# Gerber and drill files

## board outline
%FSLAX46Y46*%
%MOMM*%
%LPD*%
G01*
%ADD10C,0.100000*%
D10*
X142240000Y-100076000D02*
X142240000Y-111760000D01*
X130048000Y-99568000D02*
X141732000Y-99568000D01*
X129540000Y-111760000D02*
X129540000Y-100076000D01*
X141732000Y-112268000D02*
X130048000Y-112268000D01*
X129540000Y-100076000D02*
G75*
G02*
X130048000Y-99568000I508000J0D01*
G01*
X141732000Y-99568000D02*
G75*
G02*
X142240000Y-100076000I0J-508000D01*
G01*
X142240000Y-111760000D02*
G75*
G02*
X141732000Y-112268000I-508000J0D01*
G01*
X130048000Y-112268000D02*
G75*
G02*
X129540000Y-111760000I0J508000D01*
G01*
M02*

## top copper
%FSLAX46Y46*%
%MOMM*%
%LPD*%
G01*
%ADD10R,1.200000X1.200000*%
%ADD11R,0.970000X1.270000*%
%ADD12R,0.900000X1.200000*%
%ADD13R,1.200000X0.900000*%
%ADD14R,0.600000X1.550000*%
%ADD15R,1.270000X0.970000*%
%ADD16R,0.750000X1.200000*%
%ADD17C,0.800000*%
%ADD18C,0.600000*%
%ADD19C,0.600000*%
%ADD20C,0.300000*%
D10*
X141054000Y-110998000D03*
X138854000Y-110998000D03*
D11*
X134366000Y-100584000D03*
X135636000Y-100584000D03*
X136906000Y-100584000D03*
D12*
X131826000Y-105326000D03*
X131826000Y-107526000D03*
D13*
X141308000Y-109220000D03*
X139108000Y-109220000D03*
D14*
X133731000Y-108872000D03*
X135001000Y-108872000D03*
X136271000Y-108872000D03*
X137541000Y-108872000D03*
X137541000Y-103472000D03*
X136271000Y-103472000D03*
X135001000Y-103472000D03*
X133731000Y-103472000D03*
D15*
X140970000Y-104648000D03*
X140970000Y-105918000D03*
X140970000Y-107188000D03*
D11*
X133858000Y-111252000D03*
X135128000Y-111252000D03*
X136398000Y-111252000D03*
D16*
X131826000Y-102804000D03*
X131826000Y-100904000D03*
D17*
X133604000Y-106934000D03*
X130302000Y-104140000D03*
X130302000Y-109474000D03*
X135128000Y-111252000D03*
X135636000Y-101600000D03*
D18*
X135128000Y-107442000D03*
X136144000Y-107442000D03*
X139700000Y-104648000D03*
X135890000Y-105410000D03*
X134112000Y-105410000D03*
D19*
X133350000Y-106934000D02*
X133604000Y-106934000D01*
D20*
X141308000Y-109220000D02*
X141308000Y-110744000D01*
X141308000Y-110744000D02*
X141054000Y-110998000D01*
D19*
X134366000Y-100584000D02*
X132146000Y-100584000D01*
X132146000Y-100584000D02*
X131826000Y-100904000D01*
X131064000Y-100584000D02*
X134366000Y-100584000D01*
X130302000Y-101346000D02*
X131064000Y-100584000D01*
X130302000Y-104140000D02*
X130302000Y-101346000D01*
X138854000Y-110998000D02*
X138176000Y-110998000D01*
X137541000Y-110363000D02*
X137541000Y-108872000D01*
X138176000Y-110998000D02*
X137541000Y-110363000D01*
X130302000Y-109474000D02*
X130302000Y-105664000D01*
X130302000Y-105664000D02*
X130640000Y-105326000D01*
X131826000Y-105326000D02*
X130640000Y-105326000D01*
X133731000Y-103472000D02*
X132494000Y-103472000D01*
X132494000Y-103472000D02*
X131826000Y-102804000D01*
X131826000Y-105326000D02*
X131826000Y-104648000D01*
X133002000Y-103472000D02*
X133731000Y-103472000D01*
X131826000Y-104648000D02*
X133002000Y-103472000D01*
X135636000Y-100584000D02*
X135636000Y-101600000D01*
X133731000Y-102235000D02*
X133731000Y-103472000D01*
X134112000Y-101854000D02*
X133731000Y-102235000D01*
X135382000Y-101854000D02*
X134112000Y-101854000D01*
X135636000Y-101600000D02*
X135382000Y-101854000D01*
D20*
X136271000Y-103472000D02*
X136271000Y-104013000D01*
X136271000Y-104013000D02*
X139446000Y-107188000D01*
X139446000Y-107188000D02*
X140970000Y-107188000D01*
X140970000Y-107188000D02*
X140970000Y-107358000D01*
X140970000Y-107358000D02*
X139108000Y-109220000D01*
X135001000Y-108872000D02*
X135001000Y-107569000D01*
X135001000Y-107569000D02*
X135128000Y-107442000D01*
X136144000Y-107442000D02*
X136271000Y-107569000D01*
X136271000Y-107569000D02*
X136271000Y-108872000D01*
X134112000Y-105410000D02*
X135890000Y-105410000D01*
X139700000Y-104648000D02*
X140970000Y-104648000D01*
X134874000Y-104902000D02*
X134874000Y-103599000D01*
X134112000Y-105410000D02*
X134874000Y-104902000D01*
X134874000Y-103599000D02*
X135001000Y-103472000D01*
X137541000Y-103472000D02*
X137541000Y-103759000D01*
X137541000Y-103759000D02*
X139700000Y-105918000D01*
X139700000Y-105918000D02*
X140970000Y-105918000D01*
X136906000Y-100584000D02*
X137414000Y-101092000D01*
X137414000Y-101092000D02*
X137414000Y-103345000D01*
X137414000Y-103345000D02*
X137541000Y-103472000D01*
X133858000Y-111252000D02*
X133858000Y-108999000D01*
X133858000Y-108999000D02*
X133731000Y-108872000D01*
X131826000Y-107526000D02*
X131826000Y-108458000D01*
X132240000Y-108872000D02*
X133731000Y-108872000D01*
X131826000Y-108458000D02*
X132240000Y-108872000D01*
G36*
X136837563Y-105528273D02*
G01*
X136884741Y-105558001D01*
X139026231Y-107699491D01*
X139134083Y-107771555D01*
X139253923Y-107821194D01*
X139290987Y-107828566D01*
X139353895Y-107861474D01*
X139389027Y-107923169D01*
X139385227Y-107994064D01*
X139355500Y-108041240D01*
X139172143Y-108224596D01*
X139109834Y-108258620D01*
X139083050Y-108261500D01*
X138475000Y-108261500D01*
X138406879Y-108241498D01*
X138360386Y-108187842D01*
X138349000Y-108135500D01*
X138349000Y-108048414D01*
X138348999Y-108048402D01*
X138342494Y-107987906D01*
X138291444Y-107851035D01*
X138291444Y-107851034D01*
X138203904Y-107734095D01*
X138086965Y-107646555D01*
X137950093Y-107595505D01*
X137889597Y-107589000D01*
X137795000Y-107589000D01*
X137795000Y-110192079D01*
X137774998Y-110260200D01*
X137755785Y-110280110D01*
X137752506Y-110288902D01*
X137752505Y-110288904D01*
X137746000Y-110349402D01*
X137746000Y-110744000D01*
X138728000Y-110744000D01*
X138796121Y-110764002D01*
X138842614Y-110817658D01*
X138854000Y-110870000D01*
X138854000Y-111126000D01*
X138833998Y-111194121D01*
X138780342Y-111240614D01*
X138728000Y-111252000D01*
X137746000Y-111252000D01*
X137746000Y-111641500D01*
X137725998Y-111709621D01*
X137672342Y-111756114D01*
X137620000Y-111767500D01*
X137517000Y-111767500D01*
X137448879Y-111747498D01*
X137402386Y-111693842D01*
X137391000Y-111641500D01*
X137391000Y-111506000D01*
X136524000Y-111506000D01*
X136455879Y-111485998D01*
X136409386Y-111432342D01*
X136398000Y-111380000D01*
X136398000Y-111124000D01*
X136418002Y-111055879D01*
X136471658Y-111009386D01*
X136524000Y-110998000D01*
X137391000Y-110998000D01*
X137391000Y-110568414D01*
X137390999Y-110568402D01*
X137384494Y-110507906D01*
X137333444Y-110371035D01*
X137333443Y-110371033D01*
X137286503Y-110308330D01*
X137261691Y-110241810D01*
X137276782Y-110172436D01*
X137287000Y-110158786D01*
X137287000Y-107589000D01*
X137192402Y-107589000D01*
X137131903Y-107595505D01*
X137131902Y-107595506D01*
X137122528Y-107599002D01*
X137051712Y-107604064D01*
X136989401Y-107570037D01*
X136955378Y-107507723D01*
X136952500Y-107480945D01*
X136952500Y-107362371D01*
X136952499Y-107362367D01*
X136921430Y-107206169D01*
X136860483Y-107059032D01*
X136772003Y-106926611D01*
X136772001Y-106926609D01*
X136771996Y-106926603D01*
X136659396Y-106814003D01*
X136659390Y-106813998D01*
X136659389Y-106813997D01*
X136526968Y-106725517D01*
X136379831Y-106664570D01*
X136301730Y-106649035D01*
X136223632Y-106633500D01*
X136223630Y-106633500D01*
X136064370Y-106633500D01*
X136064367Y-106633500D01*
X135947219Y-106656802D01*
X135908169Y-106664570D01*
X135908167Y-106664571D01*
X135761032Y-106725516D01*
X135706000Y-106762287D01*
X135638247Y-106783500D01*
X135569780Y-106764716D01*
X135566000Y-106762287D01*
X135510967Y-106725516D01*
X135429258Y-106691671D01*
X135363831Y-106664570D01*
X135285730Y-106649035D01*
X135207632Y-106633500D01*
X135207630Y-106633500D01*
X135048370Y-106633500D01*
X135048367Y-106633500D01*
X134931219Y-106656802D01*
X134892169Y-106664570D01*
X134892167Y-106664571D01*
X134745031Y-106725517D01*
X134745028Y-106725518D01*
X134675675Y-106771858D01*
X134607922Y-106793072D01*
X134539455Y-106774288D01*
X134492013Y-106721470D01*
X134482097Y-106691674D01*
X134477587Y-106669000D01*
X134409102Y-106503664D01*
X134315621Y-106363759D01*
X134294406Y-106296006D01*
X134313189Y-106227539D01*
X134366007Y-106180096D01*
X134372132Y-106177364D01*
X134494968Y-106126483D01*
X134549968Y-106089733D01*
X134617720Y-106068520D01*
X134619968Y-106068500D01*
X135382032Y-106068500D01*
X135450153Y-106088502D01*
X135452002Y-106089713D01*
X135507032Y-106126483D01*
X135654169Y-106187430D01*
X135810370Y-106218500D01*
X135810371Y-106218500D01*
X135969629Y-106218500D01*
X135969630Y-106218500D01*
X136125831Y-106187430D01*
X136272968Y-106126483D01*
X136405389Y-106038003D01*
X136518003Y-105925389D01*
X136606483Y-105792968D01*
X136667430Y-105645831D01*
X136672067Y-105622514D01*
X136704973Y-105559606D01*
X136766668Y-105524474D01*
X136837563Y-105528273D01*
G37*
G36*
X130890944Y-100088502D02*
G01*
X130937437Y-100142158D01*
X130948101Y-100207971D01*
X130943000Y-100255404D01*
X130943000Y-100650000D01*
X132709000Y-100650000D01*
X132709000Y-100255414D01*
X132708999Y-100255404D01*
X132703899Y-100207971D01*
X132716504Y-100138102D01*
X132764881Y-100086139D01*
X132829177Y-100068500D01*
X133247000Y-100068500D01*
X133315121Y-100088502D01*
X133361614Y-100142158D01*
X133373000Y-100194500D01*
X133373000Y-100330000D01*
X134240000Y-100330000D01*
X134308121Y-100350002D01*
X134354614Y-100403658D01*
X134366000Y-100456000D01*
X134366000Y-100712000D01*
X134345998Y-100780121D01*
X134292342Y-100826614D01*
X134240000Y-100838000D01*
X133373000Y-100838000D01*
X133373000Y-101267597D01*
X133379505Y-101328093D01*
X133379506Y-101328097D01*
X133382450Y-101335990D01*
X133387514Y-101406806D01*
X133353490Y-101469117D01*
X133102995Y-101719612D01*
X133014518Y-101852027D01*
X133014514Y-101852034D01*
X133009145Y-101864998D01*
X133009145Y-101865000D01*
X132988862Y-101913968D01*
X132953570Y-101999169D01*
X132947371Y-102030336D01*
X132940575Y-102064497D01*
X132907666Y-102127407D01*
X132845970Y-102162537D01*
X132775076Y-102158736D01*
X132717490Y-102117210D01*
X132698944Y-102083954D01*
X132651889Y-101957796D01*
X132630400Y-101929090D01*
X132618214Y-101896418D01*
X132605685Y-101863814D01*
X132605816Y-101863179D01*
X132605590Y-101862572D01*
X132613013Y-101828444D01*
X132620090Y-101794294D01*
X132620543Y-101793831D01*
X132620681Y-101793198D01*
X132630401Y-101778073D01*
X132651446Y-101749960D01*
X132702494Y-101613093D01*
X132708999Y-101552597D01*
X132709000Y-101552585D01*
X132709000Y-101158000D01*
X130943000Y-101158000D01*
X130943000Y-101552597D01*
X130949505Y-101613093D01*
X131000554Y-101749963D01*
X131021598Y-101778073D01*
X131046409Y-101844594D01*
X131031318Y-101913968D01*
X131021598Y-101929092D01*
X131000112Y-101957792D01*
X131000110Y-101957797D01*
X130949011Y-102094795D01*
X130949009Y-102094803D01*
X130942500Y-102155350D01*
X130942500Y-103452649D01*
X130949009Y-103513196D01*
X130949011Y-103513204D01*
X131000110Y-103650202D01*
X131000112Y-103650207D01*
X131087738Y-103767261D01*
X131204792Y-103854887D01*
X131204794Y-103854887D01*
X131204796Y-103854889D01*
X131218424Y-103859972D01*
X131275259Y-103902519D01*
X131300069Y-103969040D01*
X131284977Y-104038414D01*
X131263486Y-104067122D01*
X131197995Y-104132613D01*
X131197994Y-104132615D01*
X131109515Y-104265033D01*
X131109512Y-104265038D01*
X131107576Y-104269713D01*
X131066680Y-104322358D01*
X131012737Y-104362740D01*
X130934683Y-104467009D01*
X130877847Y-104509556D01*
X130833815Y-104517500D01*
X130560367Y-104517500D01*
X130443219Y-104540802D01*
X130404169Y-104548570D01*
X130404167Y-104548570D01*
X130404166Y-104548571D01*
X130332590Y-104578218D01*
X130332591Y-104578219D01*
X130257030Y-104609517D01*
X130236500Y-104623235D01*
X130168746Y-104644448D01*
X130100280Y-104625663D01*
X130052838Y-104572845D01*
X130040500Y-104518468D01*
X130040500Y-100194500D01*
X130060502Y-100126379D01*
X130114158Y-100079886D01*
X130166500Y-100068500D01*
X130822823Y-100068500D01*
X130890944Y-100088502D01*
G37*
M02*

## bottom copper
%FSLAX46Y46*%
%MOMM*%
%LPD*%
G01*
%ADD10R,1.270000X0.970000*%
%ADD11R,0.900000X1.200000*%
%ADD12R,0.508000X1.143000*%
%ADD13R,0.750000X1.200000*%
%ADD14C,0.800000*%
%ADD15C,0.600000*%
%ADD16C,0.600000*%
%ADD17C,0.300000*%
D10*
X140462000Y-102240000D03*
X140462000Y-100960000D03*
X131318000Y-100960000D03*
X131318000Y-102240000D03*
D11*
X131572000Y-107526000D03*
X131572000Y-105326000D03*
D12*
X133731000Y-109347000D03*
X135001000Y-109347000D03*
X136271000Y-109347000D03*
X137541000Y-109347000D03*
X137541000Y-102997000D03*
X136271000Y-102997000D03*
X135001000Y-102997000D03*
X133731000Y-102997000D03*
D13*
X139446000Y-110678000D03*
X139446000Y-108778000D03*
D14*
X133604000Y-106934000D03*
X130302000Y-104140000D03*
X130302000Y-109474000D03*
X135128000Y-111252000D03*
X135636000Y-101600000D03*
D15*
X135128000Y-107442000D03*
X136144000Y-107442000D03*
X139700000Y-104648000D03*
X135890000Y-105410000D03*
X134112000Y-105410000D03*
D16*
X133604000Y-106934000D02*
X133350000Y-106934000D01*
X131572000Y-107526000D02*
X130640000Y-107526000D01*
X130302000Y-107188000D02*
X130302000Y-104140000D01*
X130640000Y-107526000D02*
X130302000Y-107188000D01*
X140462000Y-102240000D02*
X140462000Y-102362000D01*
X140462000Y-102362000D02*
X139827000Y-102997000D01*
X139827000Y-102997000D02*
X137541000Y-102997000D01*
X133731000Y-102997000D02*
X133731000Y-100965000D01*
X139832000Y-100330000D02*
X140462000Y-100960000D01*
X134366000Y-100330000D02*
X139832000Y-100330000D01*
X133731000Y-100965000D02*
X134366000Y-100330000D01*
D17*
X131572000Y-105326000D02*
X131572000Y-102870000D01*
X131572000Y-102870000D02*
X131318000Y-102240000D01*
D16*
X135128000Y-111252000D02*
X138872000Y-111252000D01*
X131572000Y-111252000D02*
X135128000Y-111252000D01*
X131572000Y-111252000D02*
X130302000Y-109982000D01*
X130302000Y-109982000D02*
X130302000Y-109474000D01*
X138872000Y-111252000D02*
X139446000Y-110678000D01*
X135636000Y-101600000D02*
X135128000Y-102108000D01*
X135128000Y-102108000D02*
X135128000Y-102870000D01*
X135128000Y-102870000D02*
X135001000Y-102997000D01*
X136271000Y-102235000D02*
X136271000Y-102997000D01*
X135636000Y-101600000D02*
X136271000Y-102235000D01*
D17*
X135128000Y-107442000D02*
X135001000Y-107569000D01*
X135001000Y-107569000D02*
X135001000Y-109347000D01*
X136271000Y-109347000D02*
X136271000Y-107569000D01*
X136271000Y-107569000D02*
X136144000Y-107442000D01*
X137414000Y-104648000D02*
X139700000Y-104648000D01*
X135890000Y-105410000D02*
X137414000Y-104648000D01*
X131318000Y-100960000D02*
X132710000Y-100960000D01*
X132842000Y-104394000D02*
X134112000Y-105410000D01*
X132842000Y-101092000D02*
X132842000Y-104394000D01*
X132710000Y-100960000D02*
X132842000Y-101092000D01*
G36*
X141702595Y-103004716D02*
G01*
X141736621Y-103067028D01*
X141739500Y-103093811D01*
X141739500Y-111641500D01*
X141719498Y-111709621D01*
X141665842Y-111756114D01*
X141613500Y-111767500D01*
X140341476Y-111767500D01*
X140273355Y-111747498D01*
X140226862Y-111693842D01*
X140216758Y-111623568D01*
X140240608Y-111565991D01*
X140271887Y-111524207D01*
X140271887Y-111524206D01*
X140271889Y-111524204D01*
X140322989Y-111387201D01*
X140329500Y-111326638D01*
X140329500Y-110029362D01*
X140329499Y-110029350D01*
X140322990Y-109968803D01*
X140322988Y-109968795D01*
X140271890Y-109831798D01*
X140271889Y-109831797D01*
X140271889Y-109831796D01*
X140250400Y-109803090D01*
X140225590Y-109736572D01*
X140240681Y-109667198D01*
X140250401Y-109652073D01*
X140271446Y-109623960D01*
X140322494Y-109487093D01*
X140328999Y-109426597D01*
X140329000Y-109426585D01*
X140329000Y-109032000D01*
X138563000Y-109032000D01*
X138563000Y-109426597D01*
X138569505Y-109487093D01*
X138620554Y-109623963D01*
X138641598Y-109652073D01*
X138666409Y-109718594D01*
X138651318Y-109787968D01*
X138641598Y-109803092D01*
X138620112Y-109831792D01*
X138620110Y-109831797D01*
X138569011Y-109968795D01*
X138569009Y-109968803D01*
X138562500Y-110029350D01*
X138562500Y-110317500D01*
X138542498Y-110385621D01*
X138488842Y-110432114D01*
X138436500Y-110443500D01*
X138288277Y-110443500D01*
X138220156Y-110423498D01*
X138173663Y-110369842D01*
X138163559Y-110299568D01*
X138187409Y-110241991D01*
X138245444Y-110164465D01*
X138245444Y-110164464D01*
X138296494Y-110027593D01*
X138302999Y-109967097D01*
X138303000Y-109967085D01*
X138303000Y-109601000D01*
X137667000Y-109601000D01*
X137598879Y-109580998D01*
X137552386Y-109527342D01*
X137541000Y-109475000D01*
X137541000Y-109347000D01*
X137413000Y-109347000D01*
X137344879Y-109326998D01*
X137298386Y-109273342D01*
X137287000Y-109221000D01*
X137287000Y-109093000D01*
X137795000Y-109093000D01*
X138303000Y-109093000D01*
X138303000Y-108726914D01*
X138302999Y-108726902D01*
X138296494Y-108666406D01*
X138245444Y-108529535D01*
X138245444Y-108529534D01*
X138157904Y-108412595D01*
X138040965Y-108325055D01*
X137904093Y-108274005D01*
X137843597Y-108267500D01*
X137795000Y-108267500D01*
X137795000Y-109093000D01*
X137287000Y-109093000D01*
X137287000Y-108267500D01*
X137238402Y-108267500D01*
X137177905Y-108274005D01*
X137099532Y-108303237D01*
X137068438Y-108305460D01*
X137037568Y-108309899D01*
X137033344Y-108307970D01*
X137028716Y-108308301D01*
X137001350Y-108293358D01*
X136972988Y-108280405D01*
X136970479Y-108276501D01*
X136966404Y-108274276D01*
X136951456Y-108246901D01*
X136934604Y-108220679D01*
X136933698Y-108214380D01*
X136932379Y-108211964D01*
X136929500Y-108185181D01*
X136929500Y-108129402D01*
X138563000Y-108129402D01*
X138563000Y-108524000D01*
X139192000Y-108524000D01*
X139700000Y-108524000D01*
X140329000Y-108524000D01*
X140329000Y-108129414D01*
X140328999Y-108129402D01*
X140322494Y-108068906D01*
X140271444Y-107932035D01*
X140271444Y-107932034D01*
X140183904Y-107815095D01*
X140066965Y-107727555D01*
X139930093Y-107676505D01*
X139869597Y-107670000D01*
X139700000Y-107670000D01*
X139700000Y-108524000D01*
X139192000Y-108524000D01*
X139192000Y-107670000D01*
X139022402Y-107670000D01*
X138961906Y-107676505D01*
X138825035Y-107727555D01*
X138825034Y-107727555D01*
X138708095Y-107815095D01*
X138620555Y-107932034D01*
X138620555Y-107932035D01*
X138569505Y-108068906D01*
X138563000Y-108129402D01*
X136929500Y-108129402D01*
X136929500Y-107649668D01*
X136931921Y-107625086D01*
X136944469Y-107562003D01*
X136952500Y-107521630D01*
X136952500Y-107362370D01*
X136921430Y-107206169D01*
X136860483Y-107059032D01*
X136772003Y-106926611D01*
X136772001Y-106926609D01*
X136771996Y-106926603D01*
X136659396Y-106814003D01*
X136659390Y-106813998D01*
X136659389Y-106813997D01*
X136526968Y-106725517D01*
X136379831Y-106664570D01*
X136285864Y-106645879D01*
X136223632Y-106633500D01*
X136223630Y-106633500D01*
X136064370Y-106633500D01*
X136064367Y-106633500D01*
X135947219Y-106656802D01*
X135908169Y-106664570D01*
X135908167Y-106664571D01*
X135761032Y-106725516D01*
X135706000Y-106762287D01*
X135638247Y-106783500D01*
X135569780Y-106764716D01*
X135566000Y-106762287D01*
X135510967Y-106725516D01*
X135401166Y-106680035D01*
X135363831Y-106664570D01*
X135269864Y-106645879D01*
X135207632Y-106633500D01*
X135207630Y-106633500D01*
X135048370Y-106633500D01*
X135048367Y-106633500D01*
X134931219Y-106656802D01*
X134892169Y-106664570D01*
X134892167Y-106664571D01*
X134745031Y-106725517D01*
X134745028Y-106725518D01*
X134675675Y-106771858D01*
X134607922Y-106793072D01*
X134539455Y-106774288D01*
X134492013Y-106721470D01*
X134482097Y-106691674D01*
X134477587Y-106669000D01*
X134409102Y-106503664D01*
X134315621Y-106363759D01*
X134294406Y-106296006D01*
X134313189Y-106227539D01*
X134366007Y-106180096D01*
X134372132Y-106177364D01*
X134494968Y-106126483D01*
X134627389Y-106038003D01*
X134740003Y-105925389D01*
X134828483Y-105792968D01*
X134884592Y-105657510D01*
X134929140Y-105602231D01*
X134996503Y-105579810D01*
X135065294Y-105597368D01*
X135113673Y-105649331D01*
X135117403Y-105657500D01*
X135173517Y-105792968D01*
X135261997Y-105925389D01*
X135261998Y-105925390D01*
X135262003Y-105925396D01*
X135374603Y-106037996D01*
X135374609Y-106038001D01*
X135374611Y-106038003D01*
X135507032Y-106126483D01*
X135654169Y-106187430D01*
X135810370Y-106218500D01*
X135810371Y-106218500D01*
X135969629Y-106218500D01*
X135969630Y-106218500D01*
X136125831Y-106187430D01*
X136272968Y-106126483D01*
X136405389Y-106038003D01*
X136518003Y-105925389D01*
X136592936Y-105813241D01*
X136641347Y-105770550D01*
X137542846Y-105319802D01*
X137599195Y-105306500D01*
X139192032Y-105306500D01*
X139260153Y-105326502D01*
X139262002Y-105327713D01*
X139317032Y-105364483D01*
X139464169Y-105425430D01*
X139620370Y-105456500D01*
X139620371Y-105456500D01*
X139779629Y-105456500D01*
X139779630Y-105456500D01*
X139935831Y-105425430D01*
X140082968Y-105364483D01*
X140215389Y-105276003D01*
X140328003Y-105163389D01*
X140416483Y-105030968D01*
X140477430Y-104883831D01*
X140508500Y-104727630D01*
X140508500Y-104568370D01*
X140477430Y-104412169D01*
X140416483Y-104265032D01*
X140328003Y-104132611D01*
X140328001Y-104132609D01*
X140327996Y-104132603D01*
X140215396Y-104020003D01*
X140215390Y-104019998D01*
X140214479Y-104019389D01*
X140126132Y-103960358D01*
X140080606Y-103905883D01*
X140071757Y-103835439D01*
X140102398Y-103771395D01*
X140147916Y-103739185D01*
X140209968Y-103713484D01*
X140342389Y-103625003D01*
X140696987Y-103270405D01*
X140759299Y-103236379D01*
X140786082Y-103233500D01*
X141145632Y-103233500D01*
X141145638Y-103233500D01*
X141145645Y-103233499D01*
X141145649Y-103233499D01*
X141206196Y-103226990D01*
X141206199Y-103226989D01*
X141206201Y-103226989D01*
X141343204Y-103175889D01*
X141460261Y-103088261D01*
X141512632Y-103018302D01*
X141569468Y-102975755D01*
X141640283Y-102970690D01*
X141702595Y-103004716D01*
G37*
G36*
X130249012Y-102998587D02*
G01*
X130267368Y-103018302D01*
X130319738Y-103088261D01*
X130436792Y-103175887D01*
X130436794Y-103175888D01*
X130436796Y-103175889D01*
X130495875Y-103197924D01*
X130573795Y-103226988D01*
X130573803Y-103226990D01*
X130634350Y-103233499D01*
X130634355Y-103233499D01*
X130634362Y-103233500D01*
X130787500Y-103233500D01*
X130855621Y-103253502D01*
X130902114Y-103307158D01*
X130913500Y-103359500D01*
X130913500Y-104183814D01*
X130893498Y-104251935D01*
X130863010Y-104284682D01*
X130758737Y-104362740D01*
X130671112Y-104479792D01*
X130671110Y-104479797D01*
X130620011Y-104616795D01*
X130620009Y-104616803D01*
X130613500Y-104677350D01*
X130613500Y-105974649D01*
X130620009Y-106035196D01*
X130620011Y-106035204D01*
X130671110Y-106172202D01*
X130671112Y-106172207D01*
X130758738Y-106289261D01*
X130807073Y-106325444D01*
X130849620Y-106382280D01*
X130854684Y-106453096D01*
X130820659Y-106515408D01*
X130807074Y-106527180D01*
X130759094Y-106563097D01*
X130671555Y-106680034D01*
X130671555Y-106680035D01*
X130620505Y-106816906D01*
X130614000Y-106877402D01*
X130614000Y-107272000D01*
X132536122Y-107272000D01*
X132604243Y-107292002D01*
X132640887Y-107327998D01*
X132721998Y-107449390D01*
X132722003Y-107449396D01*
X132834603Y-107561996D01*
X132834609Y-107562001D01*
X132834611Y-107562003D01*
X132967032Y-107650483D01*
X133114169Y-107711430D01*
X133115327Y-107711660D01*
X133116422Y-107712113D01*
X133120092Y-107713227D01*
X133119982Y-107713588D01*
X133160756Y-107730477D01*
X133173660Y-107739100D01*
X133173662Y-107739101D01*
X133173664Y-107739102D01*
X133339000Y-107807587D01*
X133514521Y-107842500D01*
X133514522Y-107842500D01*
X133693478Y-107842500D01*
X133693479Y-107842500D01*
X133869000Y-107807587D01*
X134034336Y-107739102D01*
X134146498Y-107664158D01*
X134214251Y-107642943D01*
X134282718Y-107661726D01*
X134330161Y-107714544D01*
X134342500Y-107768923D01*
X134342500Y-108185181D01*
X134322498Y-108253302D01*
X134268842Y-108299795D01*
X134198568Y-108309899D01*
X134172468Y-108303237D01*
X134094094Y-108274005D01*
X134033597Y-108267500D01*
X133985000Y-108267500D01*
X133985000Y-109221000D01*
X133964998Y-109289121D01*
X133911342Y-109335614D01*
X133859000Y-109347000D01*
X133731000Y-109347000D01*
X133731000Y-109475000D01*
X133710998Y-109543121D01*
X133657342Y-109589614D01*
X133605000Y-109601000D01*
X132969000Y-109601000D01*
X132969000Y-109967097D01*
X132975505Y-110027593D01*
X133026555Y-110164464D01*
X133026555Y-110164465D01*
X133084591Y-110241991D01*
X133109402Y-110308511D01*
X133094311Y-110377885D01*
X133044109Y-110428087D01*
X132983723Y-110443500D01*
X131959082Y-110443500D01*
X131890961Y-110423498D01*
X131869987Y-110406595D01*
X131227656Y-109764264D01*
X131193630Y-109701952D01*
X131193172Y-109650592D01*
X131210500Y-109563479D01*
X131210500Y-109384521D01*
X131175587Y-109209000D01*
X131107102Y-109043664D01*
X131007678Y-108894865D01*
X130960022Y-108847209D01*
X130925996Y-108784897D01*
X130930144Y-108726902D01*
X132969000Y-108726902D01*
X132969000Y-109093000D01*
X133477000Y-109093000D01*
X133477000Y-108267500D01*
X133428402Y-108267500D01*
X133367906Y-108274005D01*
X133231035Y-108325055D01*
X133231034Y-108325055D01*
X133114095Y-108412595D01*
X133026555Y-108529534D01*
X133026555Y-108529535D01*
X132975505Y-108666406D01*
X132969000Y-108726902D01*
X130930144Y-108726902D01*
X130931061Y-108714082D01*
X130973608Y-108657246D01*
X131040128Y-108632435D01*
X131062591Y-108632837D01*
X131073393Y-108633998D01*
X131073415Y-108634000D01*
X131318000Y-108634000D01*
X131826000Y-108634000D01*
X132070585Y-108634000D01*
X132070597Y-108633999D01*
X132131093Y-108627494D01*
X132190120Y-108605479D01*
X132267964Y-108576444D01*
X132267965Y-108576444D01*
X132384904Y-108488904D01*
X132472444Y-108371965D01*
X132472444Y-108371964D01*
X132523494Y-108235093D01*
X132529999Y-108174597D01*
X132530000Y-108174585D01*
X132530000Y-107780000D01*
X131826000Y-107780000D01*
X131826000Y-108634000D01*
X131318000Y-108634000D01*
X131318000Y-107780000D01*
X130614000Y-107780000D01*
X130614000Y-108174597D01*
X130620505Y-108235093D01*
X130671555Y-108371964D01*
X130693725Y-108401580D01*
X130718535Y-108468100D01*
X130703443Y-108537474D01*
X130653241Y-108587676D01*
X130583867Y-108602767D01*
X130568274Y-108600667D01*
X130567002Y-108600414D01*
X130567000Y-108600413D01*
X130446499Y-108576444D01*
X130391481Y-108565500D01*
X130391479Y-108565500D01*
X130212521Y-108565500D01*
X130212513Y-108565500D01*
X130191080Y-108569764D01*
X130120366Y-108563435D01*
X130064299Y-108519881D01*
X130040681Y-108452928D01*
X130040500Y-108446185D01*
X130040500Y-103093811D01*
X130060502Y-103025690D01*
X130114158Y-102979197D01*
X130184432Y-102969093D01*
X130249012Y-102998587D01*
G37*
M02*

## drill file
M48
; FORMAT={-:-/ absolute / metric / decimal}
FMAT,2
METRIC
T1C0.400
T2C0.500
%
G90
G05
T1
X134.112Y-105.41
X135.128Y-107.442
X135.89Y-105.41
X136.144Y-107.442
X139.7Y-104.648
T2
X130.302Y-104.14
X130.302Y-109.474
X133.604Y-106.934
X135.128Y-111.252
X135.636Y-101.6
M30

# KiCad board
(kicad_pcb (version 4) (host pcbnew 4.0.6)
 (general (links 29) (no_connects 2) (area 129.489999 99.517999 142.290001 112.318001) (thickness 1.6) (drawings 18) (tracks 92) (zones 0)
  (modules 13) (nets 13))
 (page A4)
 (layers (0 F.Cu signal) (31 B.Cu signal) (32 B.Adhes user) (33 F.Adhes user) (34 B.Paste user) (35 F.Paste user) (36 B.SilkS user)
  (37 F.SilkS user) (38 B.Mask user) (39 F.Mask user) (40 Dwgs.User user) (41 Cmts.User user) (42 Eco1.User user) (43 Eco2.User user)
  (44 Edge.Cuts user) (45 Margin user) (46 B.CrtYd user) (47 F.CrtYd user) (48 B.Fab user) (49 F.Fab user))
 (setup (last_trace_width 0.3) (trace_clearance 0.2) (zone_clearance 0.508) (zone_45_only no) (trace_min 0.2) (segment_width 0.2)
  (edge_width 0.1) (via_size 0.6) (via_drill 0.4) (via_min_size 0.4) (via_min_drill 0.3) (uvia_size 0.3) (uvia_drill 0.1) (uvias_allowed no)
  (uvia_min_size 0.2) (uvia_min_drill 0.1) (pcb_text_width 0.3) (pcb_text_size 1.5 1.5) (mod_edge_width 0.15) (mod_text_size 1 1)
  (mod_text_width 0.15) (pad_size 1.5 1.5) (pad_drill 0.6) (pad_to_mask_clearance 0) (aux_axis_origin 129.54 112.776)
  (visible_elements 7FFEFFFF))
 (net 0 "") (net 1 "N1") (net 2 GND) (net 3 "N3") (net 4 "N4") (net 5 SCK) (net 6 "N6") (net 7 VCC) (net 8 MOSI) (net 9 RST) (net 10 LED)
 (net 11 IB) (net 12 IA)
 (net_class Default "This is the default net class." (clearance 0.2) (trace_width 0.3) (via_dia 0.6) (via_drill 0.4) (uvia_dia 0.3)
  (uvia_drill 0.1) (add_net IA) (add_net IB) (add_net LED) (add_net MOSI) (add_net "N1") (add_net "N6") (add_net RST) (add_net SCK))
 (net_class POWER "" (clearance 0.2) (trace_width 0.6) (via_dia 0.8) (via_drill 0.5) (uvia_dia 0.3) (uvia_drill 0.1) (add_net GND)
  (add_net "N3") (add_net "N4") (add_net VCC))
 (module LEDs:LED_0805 (layer F.Cu) (at 139.954 110.998)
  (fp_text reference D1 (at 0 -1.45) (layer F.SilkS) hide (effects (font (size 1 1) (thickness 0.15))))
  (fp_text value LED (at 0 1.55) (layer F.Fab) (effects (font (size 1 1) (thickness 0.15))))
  (pad 2 smd rect (at 1.1 0 180) (size 1.2 1.2) (layers F.Cu F.Paste F.Mask) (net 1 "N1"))
  (pad 1 smd rect (at -1.1 0 180) (size 1.2 1.2) (layers F.Cu F.Paste F.Mask) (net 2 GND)))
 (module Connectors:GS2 (layer B.Cu) (at 140.462 101.6)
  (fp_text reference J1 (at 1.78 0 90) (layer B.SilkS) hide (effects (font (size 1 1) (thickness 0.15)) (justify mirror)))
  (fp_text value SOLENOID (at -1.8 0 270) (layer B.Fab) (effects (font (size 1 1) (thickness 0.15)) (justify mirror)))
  (pad 1 smd rect (at 0 0.64) (size 1.27 0.97) (layers B.Cu B.Paste B.Mask) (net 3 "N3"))
  (pad 2 smd rect (at 0 -0.64) (size 1.27 0.97) (layers B.Cu B.Paste B.Mask) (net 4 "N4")))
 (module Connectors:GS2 (layer B.Cu) (at 131.318 101.6 180)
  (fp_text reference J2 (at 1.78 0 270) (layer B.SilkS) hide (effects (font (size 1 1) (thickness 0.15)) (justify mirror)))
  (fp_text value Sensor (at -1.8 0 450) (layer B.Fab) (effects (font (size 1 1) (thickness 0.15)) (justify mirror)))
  (pad 1 smd rect (at 0 0.64 180) (size 1.27 0.97) (layers B.Cu B.Paste B.Mask) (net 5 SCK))
  (pad 2 smd rect (at 0 -0.64 180) (size 1.27 0.97) (layers B.Cu B.Paste B.Mask) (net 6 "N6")))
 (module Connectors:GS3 (layer F.Cu) (at 135.636 100.584 90)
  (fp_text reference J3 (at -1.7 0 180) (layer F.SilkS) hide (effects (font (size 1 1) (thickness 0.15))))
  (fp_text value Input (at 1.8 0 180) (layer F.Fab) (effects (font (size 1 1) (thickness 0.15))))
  (pad 1 smd rect (at 0 -1.27 90) (size 1.27 0.97) (layers F.Cu F.Paste F.Mask) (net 2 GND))
  (pad 2 smd rect (at 0 0 90) (size 1.27 0.97) (layers F.Cu F.Paste F.Mask) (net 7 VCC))
  (pad 3 smd rect (at 0 1.27 90) (size 1.27 0.97) (layers F.Cu F.Paste F.Mask) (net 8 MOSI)))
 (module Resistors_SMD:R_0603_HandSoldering (layer F.Cu) (at 131.826 106.426 270)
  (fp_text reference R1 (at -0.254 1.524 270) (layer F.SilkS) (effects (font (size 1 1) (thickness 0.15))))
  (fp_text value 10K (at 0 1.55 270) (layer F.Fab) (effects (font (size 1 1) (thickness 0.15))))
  (pad 1 smd rect (at -1.1 0 270) (size 1.2 0.9) (layers F.Cu F.Paste F.Mask) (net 7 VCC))
  (pad 2 smd rect (at 1.1 0 270) (size 1.2 0.9) (layers F.Cu F.Paste F.Mask) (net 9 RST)))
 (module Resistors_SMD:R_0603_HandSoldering (layer B.Cu) (at 131.572 106.426 90)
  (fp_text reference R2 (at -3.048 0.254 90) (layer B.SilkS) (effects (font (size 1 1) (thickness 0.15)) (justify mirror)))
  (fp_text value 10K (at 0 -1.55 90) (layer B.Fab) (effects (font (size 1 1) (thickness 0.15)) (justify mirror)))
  (pad 1 smd rect (at -1.1 0 90) (size 1.2 0.9) (layers B.Cu B.Paste B.Mask) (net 2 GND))
  (pad 2 smd rect (at 1.1 0 90) (size 1.2 0.9) (layers B.Cu B.Paste B.Mask) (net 6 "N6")))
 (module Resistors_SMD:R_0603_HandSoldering (layer F.Cu) (at 140.208 109.22 180)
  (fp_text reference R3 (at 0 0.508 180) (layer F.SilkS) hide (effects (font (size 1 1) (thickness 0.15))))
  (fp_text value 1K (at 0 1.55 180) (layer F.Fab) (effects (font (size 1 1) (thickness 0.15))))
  (pad 1 smd rect (at -1.1 0 180) (size 1.2 0.9) (layers F.Cu F.Paste F.Mask) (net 1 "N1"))
  (pad 2 smd rect (at 1.1 0 180) (size 1.2 0.9) (layers F.Cu F.Paste F.Mask) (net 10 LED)))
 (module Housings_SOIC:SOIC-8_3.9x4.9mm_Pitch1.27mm (layer F.Cu) (at 135.636 106.172 90)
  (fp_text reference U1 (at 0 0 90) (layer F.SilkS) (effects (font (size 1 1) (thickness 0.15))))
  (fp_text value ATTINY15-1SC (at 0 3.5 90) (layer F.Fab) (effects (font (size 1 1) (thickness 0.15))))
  (pad 1 smd rect (at -2.7 -1.905 90) (size 1.55 0.6) (layers F.Cu F.Paste F.Mask) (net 9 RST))
  (pad 2 smd rect (at -2.7 -0.635 90) (size 1.55 0.6) (layers F.Cu F.Paste F.Mask) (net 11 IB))
  (pad 3 smd rect (at -2.7 0.635 90) (size 1.55 0.6) (layers F.Cu F.Paste F.Mask) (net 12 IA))
  (pad 4 smd rect (at -2.7 1.905 90) (size 1.55 0.6) (layers F.Cu F.Paste F.Mask) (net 2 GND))
  (pad 5 smd rect (at 2.7 1.905 90) (size 1.55 0.6) (layers F.Cu F.Paste F.Mask) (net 8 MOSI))
  (pad 6 smd rect (at 2.7 0.635 90) (size 1.55 0.6) (layers F.Cu F.Paste F.Mask) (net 10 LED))
  (pad 7 smd rect (at 2.7 -0.635 90) (size 1.55 0.6) (layers F.Cu F.Paste F.Mask) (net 5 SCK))
  (pad 8 smd rect (at 2.7 -1.905 90) (size 1.55 0.6) (layers F.Cu F.Paste F.Mask) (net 7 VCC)))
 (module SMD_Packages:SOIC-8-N (layer B.Cu) (at 135.636 106.172)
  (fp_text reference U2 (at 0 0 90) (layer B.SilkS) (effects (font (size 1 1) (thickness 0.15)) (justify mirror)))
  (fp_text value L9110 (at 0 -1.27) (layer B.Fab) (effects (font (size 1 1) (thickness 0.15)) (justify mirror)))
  (pad 8 smd rect (at -1.905 3.175) (size 0.508 1.143) (layers B.Cu B.Paste B.Mask) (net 2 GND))
  (pad 7 smd rect (at -0.635 3.175) (size 0.508 1.143) (layers B.Cu B.Paste B.Mask) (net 11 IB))
  (pad 6 smd rect (at 0.635 3.175) (size 0.508 1.143) (layers B.Cu B.Paste B.Mask) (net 12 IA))
  (pad 5 smd rect (at 1.905 3.175) (size 0.508 1.143) (layers B.Cu B.Paste B.Mask) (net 2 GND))
  (pad 4 smd rect (at 1.905 -3.175) (size 0.508 1.143) (layers B.Cu B.Paste B.Mask) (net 3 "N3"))
  (pad 3 smd rect (at 0.635 -3.175) (size 0.508 1.143) (layers B.Cu B.Paste B.Mask) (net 7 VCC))
  (pad 2 smd rect (at -0.635 -3.175) (size 0.508 1.143) (layers B.Cu B.Paste B.Mask) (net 7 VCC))
  (pad 1 smd rect (at -1.905 -3.175) (size 0.508 1.143) (layers B.Cu B.Paste B.Mask) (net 4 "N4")))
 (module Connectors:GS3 (layer F.Cu) (at 140.97 105.918)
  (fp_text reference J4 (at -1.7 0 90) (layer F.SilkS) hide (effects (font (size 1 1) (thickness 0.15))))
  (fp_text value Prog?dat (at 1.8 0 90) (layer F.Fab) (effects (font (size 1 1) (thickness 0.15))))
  (pad 1 smd rect (at 0 -1.27) (size 1.27 0.97) (layers F.Cu F.Paste F.Mask) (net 5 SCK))
  (pad 2 smd rect (at 0 0) (size 1.27 0.97) (layers F.Cu F.Paste F.Mask) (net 8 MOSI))
  (pad 3 smd rect (at 0 1.27) (size 1.27 0.97) (layers F.Cu F.Paste F.Mask) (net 10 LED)))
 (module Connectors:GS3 (layer F.Cu) (at 135.128 111.252 90)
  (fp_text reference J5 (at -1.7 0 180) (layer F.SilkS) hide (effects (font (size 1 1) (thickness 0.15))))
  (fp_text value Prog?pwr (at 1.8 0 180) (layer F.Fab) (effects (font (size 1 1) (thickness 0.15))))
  (pad 1 smd rect (at 0 -1.27 90) (size 1.27 0.97) (layers F.Cu F.Paste F.Mask) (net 9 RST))
  (pad 2 smd rect (at 0 0 90) (size 1.27 0.97) (layers F.Cu F.Paste F.Mask) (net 7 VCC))
  (pad 3 smd rect (at 0 1.27 90) (size 1.27 0.97) (layers F.Cu F.Paste F.Mask) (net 2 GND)))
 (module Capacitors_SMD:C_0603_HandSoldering (layer B.Cu) (at 139.446 109.728 90)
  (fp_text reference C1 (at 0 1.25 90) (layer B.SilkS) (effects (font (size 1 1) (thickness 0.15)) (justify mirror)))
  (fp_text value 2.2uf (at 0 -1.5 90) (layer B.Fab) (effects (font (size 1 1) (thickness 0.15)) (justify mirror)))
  (pad 1 smd rect (at -0.95 0 90) (size 1.2 0.75) (layers B.Cu B.Paste B.Mask) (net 7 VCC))
  (pad 2 smd rect (at 0.95 0 90) (size 1.2 0.75) (layers B.Cu B.Paste B.Mask) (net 2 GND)))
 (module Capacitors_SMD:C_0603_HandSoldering (layer F.Cu) (at 131.826 101.854 90)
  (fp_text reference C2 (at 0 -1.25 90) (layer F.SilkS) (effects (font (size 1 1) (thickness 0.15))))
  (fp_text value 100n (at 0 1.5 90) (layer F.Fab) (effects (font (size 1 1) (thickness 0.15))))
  (pad 1 smd rect (at -0.95 0 90) (size 1.2 0.75) (layers F.Cu F.Paste F.Mask) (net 7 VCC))
  (pad 2 smd rect (at 0.95 0 90) (size 1.2 0.75) (layers F.Cu F.Paste F.Mask) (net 2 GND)))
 (gr_line (start 142.24 100.076) (end 142.24 111.76) (angle 90) (layer Edge.Cuts) (width 0.1))
 (gr_line (start 130.048 99.568) (end 141.732 99.568) (angle 90) (layer Edge.Cuts) (width 0.1))
 (gr_line (start 129.54 111.76) (end 129.54 100.076) (angle 90) (layer Edge.Cuts) (width 0.1))
 (gr_line (start 141.732 112.268) (end 130.048 112.268) (angle 90) (layer Edge.Cuts) (width 0.1))
 (gr_arc (start 130.048 100.076) (end 129.54 100.076) (angle 90) (layer Edge.Cuts) (width 0.1))
 (gr_arc (start 141.732 100.076) (end 141.732 99.568) (angle 90) (layer Edge.Cuts) (width 0.1))
 (gr_arc (start 141.732 111.76) (end 142.24 111.76) (angle 90) (layer Edge.Cuts) (width 0.1))
 (gr_arc (start 130.048 111.76) (end 130.048 112.268) (angle 90) (layer Edge.Cuts) (width 0.1))
 (segment (start 133.35 106.934) (end 133.604 106.934) (width 0.6) (layer F.Cu) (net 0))
 (segment (start 133.604 106.934) (end 133.35 106.934) (width 0.6) (layer B.Cu) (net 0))
 (via (at 133.604 106.934) (size 0.8) (drill 0.5) (layers F.Cu B.Cu) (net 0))
 (segment (start 141.308 109.22) (end 141.308 110.744) (width 0.3) (layer F.Cu) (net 1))
 (segment (start 141.308 110.744) (end 141.054 110.998) (width 0.3) (layer F.Cu) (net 1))
 (segment (start 134.366 100.584) (end 132.146 100.584) (width 0.6) (layer F.Cu) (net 2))
 (segment (start 132.146 100.584) (end 131.826 100.904) (width 0.6) (layer F.Cu) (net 2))
 (segment (start 131.572 107.526) (end 130.64 107.526) (width 0.6) (layer B.Cu) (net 2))
 (segment (start 131.064 100.584) (end 134.366 100.584) (width 0.6) (layer F.Cu) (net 2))
 (segment (start 130.302 101.346) (end 131.064 100.584) (width 0.6) (layer F.Cu) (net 2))
 (segment (start 130.302 104.14) (end 130.302 101.346) (width 0.6) (layer F.Cu) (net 2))
 (via (at 130.302 104.14) (size 0.8) (drill 0.5) (layers F.Cu B.Cu) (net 2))
 (segment (start 130.302 107.188) (end 130.302 104.14) (width 0.6) (layer B.Cu) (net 2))
 (segment (start 130.64 107.526) (end 130.302 107.188) (width 0.6) (layer B.Cu) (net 2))
 (segment (start 138.854 110.998) (end 138.176 110.998) (width 0.6) (layer F.Cu) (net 2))
 (segment (start 137.541 110.363) (end 137.541 108.872) (width 0.6) (layer F.Cu) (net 2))
 (segment (start 138.176 110.998) (end 137.541 110.363) (width 0.6) (layer F.Cu) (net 2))
 (segment (start 140.462 102.24) (end 140.462 102.362) (width 0.6) (layer B.Cu) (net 3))
 (segment (start 140.462 102.362) (end 139.827 102.997) (width 0.6) (layer B.Cu) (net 3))
 (segment (start 139.827 102.997) (end 137.541 102.997) (width 0.6) (layer B.Cu) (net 3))
 (segment (start 133.731 102.997) (end 133.731 100.965) (width 0.6) (layer B.Cu) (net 4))
 (segment (start 139.832 100.33) (end 140.462 100.96) (width 0.6) (layer B.Cu) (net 4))
 (segment (start 134.366 100.33) (end 139.832 100.33) (width 0.6) (layer B.Cu) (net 4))
 (segment (start 133.731 100.965) (end 134.366 100.33) (width 0.6) (layer B.Cu) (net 4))
 (segment (start 131.572 105.326) (end 131.572 102.87) (width 0.3) (layer B.Cu) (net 6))
 (segment (start 131.572 102.87) (end 131.318 102.24) (width 0.3) (layer B.Cu) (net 6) (status 20))
 (segment (start 135.128 111.252) (end 138.872 111.252) (width 0.6) (layer B.Cu) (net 7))
 (segment (start 131.572 111.252) (end 135.128 111.252) (width 0.6) (layer B.Cu) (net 7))
 (segment (start 131.572 111.252) (end 130.302 109.982) (width 0.6) (layer B.Cu) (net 7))
 (segment (start 130.302 109.982) (end 130.302 109.474) (width 0.6) (layer B.Cu) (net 7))
 (via (at 130.302 109.474) (size 0.8) (drill 0.5) (layers F.Cu B.Cu) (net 7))
 (segment (start 130.302 109.474) (end 130.302 105.664) (width 0.6) (layer F.Cu) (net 7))
 (segment (start 130.302 105.664) (end 130.64 105.326) (width 0.6) (layer F.Cu) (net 7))
 (segment (start 131.826 105.326) (end 130.64 105.326) (width 0.6) (layer F.Cu) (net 7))
 (via (at 135.128 111.252) (size 0.8) (drill 0.5) (layers F.Cu B.Cu) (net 7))
 (segment (start 138.872 111.252) (end 139.446 110.678) (width 0.6) (layer B.Cu) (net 7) (status 800000))
 (segment (start 133.731 103.472) (end 132.494 103.472) (width 0.6) (layer F.Cu) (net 7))
 (segment (start 132.494 103.472) (end 131.826 102.804) (width 0.6) (layer F.Cu) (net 7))
 (segment (start 131.826 105.326) (end 131.826 104.648) (width 0.6) (layer F.Cu) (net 7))
 (segment (start 133.002 103.472) (end 133.731 103.472) (width 0.6) (layer F.Cu) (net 7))
 (segment (start 131.826 104.648) (end 133.002 103.472) (width 0.6) (layer F.Cu) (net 7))
 (segment (start 135.636 101.6) (end 135.128 102.108) (width 0.6) (layer B.Cu) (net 7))
 (segment (start 135.128 102.108) (end 135.128 102.87) (width 0.6) (layer B.Cu) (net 7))
 (segment (start 135.128 102.87) (end 135.001 102.997) (width 0.6) (layer B.Cu) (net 7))
 (segment (start 135.636 100.584) (end 135.636 101.6) (width 0.6) (layer F.Cu) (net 7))
 (via (at 135.636 101.6) (size 0.8) (drill 0.5) (layers F.Cu B.Cu) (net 7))
 (segment (start 136.271 102.235) (end 136.271 102.997) (width 0.6) (layer B.Cu) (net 7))
 (segment (start 135.636 101.6) (end 136.271 102.235) (width 0.6) (layer B.Cu) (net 7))
 (segment (start 133.731 102.235) (end 133.731 103.472) (width 0.6) (layer F.Cu) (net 7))
 (segment (start 134.112 101.854) (end 133.731 102.235) (width 0.6) (layer F.Cu) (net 7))
 (segment (start 135.382 101.854) (end 134.112 101.854) (width 0.6) (layer F.Cu) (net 7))
 (segment (start 135.636 101.6) (end 135.382 101.854) (width 0.6) (layer F.Cu) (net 7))
 (segment (start 136.271 103.472) (end 136.271 104.013) (width 0.3) (layer F.Cu) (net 10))
 (segment (start 136.271 104.013) (end 139.446 107.188) (width 0.3) (layer F.Cu) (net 10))
 (segment (start 139.446 107.188) (end 140.97 107.188) (width 0.3) (layer F.Cu) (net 10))
 (segment (start 140.97 107.188) (end 140.97 107.358) (width 0.3) (layer F.Cu) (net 10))
 (segment (start 140.97 107.358) (end 139.108 109.22) (width 0.3) (layer F.Cu) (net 10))
 (segment (start 135.001 108.872) (end 135.001 107.569) (width 0.3) (layer F.Cu) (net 11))
 (segment (start 135.001 107.569) (end 135.128 107.442) (width 0.3) (layer F.Cu) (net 11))
 (via (at 135.128 107.442) (size 0.6) (drill 0.4) (layers F.Cu B.Cu) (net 11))
 (segment (start 135.128 107.442) (end 135.001 107.569) (width 0.3) (layer B.Cu) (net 11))
 (segment (start 135.001 107.569) (end 135.001 109.347) (width 0.3) (layer B.Cu) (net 11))
 (segment (start 136.271 109.347) (end 136.271 107.569) (width 0.3) (layer B.Cu) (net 12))
 (segment (start 136.271 107.569) (end 136.144 107.442) (width 0.3) (layer B.Cu) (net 12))
 (via (at 136.144 107.442) (size 0.6) (drill 0.4) (layers F.Cu B.Cu) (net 12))
 (segment (start 136.144 107.442) (end 136.271 107.569) (width 0.3) (layer F.Cu) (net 12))
 (segment (start 136.271 107.569) (end 136.271 108.872) (width 0.3) (layer F.Cu) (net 12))
 (segment (start 134.112 105.41) (end 135.89 105.41) (width 0.3) (layer F.Cu) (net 5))
 (segment (start 139.7 104.648) (end 140.97 104.648) (width 0.3) (layer F.Cu) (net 5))
 (via (at 139.7 104.648) (size 0.6) (drill 0.4) (layers F.Cu B.Cu) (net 5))
 (segment (start 137.414 104.648) (end 139.7 104.648) (width 0.3) (layer B.Cu) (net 5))
 (segment (start 135.89 105.41) (end 137.414 104.648) (width 0.3) (layer B.Cu) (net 5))
 (via (at 135.89 105.41) (size 0.6) (drill 0.4) (layers F.Cu B.Cu) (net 5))
 (segment (start 131.318 100.96) (end 132.71 100.96) (width 0.3) (layer B.Cu) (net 5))
 (segment (start 134.874 104.902) (end 134.874 103.599) (width 0.3) (layer F.Cu) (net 5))
 (segment (start 134.112 105.41) (end 134.874 104.902) (width 0.3) (layer F.Cu) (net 5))
 (via (at 134.112 105.41) (size 0.6) (drill 0.4) (layers F.Cu B.Cu) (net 5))
 (segment (start 132.842 104.394) (end 134.112 105.41) (width 0.3) (layer B.Cu) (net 5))
 (segment (start 132.842 101.092) (end 132.842 104.394) (width 0.3) (layer B.Cu) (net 5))
 (segment (start 132.71 100.96) (end 132.842 101.092) (width 0.3) (layer B.Cu) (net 5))
 (segment (start 134.874 103.599) (end 135.001 103.472) (width 0.3) (layer F.Cu) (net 5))
 (segment (start 137.541 103.472) (end 137.541 103.759) (width 0.3) (layer F.Cu) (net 8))
 (segment (start 137.541 103.759) (end 139.7 105.918) (width 0.3) (layer F.Cu) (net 8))
 (segment (start 139.7 105.918) (end 140.97 105.918) (width 0.3) (layer F.Cu) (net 8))
 (segment (start 136.906 100.584) (end 137.414 101.092) (width 0.3) (layer F.Cu) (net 8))
 (segment (start 137.414 101.092) (end 137.414 103.345) (width 0.3) (layer F.Cu) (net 8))
 (segment (start 137.414 103.345) (end 137.541 103.472) (width 0.3) (layer F.Cu) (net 8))
 (segment (start 133.858 111.252) (end 133.858 108.999) (width 0.3) (layer F.Cu) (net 9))
 (segment (start 133.858 108.999) (end 133.731 108.872) (width 0.3) (layer F.Cu) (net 9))
 (segment (start 131.826 107.526) (end 131.826 108.458) (width 0.3) (layer F.Cu) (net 9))
 (segment (start 132.24 108.872) (end 133.731 108.872) (width 0.3) (layer F.Cu) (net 9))
 (segment (start 131.826 108.458) (end 132.24 108.872) (width 0.3) (layer F.Cu) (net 9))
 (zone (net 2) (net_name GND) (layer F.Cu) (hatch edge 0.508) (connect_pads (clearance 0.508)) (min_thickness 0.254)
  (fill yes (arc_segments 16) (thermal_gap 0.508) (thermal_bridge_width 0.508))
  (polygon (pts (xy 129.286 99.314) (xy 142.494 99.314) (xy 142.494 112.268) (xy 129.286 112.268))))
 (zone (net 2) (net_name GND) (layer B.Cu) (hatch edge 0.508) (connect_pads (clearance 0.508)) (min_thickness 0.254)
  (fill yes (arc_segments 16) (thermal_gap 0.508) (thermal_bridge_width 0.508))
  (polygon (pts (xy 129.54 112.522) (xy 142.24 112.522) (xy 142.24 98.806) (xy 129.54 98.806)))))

